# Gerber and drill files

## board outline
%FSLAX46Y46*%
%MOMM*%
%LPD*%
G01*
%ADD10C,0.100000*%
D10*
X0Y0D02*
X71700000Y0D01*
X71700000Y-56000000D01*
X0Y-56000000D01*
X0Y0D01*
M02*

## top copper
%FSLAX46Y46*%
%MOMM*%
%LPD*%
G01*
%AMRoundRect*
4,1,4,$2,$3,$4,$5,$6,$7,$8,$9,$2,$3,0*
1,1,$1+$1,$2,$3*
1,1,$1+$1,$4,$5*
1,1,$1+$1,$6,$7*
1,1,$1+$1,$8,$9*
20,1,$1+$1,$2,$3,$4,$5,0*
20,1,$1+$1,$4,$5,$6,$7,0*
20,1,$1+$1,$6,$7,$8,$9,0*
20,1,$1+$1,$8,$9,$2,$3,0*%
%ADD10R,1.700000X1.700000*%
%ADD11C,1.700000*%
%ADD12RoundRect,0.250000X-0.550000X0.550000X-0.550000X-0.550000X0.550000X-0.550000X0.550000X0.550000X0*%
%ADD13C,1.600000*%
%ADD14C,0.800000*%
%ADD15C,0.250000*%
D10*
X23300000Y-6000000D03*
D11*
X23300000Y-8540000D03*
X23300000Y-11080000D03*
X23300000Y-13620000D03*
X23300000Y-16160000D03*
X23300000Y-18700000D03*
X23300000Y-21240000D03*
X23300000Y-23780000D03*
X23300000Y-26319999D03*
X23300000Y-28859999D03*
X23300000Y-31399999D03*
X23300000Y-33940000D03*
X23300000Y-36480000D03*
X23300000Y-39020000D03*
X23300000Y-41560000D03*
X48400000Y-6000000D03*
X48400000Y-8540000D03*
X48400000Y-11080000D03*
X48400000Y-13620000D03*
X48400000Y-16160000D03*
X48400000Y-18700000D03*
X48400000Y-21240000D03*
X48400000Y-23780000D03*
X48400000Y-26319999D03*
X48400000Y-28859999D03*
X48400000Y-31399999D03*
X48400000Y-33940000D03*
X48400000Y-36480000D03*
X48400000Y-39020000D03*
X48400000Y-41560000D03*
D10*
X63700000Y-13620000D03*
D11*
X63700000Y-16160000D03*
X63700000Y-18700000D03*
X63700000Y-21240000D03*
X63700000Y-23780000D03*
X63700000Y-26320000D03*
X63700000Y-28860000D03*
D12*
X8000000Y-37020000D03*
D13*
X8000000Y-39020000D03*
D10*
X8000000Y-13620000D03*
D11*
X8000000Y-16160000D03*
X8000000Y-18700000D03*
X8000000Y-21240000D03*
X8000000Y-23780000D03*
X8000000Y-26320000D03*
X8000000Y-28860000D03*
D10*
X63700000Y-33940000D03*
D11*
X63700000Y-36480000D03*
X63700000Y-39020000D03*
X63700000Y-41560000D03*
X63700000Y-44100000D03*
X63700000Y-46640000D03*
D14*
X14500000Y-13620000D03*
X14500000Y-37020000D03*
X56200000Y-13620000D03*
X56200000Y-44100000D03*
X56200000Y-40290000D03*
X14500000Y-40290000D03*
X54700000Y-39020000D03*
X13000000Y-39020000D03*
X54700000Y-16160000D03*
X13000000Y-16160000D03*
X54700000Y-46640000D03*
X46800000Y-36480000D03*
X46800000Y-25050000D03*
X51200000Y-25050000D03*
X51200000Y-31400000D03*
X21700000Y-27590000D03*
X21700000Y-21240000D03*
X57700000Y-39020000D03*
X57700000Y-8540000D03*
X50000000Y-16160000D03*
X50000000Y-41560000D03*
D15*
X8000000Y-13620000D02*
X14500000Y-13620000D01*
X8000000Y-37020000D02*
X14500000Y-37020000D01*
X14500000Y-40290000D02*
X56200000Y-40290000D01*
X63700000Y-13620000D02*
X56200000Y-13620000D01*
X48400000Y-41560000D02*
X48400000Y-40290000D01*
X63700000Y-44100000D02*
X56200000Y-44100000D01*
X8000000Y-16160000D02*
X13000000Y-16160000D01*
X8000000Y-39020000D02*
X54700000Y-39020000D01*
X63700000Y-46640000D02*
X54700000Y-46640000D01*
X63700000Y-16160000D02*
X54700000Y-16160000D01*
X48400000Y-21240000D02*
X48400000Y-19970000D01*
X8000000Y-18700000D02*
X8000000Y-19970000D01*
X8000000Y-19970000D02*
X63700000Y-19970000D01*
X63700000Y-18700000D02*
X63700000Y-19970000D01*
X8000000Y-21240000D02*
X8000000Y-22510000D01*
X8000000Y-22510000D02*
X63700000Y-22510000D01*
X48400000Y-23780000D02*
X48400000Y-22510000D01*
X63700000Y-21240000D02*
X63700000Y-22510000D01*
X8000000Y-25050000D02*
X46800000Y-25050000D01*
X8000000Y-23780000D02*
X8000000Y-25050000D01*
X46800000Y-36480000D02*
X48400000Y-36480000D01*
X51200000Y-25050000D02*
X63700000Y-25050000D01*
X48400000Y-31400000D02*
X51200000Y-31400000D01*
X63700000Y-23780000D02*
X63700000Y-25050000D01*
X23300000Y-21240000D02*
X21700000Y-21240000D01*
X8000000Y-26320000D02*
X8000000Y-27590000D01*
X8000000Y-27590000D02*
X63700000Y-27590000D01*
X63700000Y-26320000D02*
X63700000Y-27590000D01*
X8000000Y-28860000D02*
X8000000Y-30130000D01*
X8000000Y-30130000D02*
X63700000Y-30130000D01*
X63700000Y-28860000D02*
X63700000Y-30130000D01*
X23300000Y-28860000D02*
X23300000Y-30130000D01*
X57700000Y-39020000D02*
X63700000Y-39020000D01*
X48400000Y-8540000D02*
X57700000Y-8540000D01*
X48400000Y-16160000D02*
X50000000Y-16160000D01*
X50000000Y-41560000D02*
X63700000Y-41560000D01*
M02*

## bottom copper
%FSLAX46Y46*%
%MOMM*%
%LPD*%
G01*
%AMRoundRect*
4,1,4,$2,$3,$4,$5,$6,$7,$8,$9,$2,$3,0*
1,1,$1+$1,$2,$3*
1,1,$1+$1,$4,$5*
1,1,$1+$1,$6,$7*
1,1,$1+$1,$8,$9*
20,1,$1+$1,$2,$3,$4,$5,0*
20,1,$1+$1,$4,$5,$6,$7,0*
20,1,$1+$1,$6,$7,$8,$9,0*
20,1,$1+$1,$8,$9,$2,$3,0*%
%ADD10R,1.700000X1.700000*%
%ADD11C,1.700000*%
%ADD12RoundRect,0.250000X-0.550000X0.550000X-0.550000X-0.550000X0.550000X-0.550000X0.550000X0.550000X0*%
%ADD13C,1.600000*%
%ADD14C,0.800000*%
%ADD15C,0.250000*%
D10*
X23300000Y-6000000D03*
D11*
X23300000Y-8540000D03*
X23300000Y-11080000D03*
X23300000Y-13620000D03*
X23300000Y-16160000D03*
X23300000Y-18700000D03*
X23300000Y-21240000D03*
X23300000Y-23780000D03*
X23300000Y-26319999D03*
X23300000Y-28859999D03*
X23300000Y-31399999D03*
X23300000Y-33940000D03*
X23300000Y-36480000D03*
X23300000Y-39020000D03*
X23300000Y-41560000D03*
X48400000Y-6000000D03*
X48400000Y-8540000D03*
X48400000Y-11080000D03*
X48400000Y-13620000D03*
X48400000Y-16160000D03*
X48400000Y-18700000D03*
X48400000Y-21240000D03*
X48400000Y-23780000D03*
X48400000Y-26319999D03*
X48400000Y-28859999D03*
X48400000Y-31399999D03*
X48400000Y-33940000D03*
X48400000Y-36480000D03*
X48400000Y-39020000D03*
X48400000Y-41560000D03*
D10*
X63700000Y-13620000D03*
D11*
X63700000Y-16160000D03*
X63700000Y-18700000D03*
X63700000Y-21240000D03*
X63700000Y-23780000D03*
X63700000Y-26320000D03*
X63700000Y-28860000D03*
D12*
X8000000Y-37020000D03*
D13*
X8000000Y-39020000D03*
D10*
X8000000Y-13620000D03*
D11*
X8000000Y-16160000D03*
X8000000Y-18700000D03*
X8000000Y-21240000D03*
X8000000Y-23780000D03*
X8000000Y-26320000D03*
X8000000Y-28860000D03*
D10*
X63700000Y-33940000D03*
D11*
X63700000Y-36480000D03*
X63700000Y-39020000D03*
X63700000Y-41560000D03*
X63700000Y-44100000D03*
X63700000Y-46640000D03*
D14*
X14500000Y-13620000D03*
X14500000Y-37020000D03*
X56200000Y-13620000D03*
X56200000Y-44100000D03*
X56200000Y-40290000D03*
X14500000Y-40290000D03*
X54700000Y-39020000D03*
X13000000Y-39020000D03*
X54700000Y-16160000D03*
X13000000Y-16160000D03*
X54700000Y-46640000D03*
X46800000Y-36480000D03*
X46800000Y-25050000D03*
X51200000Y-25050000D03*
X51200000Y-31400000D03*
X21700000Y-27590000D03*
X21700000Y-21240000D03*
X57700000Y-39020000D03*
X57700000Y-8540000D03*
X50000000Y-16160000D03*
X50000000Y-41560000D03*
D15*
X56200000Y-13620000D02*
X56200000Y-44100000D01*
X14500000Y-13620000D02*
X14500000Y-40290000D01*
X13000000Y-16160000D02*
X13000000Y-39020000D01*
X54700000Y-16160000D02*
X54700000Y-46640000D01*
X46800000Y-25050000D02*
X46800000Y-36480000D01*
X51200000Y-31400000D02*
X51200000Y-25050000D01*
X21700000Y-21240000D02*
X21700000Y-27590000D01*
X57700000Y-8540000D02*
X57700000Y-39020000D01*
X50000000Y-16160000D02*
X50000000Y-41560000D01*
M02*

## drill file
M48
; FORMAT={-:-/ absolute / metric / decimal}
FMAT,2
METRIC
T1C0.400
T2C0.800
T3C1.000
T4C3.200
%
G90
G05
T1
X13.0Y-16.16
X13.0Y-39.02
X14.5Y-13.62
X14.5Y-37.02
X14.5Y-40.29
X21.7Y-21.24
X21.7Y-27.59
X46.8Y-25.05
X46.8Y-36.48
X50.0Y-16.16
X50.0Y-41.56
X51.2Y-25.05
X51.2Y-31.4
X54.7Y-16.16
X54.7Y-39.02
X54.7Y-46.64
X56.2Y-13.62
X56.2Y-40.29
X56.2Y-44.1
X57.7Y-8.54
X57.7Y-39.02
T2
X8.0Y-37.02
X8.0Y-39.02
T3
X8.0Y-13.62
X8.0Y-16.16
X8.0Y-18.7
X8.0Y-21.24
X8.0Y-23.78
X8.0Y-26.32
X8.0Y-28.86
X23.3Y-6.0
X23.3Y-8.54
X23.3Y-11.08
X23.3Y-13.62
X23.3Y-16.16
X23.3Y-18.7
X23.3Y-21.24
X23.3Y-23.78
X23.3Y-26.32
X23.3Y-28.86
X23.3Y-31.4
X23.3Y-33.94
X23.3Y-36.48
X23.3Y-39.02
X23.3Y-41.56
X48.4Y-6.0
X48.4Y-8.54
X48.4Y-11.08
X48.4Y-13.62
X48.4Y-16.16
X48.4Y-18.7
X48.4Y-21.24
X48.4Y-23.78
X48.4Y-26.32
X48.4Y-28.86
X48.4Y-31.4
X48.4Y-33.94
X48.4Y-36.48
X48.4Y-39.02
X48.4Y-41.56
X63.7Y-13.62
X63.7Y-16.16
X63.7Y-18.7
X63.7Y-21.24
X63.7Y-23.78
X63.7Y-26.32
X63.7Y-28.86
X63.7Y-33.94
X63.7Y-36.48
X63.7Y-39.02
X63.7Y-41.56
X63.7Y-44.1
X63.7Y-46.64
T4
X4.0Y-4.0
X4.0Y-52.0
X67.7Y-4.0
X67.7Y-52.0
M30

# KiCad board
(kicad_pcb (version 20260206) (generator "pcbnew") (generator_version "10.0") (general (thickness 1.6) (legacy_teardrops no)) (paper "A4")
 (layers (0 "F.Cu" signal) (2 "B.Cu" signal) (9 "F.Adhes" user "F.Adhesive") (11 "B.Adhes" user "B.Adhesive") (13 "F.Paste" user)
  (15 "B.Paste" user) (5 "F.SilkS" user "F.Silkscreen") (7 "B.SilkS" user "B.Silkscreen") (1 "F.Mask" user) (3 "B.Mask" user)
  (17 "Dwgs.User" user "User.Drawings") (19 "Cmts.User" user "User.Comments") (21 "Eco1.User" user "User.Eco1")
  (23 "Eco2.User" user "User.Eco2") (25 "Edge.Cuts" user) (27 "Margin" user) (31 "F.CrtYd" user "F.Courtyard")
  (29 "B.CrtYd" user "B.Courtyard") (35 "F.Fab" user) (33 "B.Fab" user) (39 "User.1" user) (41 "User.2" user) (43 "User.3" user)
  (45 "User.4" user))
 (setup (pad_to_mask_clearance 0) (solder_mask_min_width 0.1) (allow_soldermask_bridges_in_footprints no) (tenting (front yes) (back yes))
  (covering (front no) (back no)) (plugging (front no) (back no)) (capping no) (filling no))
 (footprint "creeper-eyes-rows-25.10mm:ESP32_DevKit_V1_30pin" (layer "F.Cu") (at 35.85 23.78)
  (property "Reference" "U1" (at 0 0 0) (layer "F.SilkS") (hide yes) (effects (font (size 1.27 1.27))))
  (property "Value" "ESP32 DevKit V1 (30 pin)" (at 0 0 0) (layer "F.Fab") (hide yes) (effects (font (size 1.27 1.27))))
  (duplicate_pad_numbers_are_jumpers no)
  (pad "1" thru_hole rect (at -12.55 -17.78) (size 1.7 1.7) (drill 1) (layers "*.Cu" "*.Mask") (remove_unused_layers no)
   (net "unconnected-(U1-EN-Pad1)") (thermal_bridge_angle 45))
  (pad "2" thru_hole circle (at -12.55 -15.24) (size 1.7 1.7) (drill 1) (layers "*.Cu" "*.Mask") (remove_unused_layers no)
   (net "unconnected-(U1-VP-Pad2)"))
  (pad "3" thru_hole circle (at -12.55 -12.7) (size 1.7 1.7) (drill 1) (layers "*.Cu" "*.Mask") (remove_unused_layers no)
   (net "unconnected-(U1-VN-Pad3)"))
  (pad "4" thru_hole circle (at -12.55 -10.16) (size 1.7 1.7) (drill 1) (layers "*.Cu" "*.Mask") (remove_unused_layers no)
   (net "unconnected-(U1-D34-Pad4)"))
  (pad "5" thru_hole circle (at -12.55 -7.62) (size 1.7 1.7) (drill 1) (layers "*.Cu" "*.Mask") (remove_unused_layers no)
   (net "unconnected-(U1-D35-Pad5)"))
  (pad "6" thru_hole circle (at -12.55 -5.08) (size 1.7 1.7) (drill 1) (layers "*.Cu" "*.Mask") (remove_unused_layers no)
   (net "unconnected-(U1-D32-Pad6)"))
  (pad "7" thru_hole circle (at -12.55 -2.54) (size 1.7 1.7) (drill 1) (layers "*.Cu" "*.Mask") (remove_unused_layers no) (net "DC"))
  (pad "8" thru_hole circle (at -12.55 0) (size 1.7 1.7) (drill 1) (layers "*.Cu" "*.Mask") (remove_unused_layers no)
   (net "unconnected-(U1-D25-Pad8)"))
  (pad "9" thru_hole circle (at -12.55 2.539999) (size 1.7 1.7) (drill 1) (layers "*.Cu" "*.Mask") (remove_unused_layers no)
   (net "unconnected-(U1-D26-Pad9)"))
  (pad "10" thru_hole circle (at -12.55 5.079999) (size 1.7 1.7) (drill 1) (layers "*.Cu" "*.Mask") (remove_unused_layers no) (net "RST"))
  (pad "11" thru_hole circle (at -12.55 7.619999) (size 1.7 1.7) (drill 1) (layers "*.Cu" "*.Mask") (remove_unused_layers no)
   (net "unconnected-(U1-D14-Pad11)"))
  (pad "12" thru_hole circle (at -12.55 10.16) (size 1.7 1.7) (drill 1) (layers "*.Cu" "*.Mask") (remove_unused_layers no)
   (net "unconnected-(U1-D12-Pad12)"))
  (pad "13" thru_hole circle (at -12.55 12.7) (size 1.7 1.7) (drill 1) (layers "*.Cu" "*.Mask") (remove_unused_layers no)
   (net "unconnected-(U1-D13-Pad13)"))
  (pad "14" thru_hole circle (at -12.55 15.24) (size 1.7 1.7) (drill 1) (layers "*.Cu" "*.Mask") (remove_unused_layers no) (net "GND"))
  (pad "15" thru_hole circle (at -12.55 17.78) (size 1.7 1.7) (drill 1) (layers "*.Cu" "*.Mask") (remove_unused_layers no)
   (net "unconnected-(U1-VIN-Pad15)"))
  (pad "16" thru_hole circle (at 12.55 -17.78) (size 1.7 1.7) (drill 1) (layers "*.Cu" "*.Mask") (remove_unused_layers no)
   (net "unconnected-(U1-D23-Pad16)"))
  (pad "17" thru_hole circle (at 12.55 -15.24) (size 1.7 1.7) (drill 1) (layers "*.Cu" "*.Mask") (remove_unused_layers no) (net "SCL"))
  (pad "18" thru_hole circle (at 12.55 -12.7) (size 1.7 1.7) (drill 1) (layers "*.Cu" "*.Mask") (remove_unused_layers no)
   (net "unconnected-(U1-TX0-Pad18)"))
  (pad "19" thru_hole circle (at 12.55 -10.16) (size 1.7 1.7) (drill 1) (layers "*.Cu" "*.Mask") (remove_unused_layers no)
   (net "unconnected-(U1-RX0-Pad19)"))
  (pad "20" thru_hole circle (at 12.55 -7.62) (size 1.7 1.7) (drill 1) (layers "*.Cu" "*.Mask") (remove_unused_layers no) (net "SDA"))
  (pad "21" thru_hole circle (at 12.55 -5.08) (size 1.7 1.7) (drill 1) (layers "*.Cu" "*.Mask") (remove_unused_layers no)
   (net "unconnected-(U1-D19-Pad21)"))
  (pad "22" thru_hole circle (at 12.55 -2.54) (size 1.7 1.7) (drill 1) (layers "*.Cu" "*.Mask") (remove_unused_layers no) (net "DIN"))
  (pad "23" thru_hole circle (at 12.55 0) (size 1.7 1.7) (drill 1) (layers "*.Cu" "*.Mask") (remove_unused_layers no) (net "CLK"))
  (pad "24" thru_hole circle (at 12.55 2.539999) (size 1.7 1.7) (drill 1) (layers "*.Cu" "*.Mask") (remove_unused_layers no)
   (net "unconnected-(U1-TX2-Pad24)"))
  (pad "25" thru_hole circle (at 12.55 5.079999) (size 1.7 1.7) (drill 1) (layers "*.Cu" "*.Mask") (remove_unused_layers no)
   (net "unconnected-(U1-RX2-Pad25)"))
  (pad "26" thru_hole circle (at 12.55 7.619999) (size 1.7 1.7) (drill 1) (layers "*.Cu" "*.Mask") (remove_unused_layers no) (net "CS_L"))
  (pad "27" thru_hole circle (at 12.55 10.16) (size 1.7 1.7) (drill 1) (layers "*.Cu" "*.Mask") (remove_unused_layers no)
   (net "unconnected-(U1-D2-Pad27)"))
  (pad "28" thru_hole circle (at 12.55 12.7) (size 1.7 1.7) (drill 1) (layers "*.Cu" "*.Mask") (remove_unused_layers no) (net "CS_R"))
  (pad "29" thru_hole circle (at 12.55 15.24) (size 1.7 1.7) (drill 1) (layers "*.Cu" "*.Mask") (remove_unused_layers no) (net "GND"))
  (pad "30" thru_hole circle (at 12.55 17.78) (size 1.7 1.7) (drill 1) (layers "*.Cu" "*.Mask") (remove_unused_layers no) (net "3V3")))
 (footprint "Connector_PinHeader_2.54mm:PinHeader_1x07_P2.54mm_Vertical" (layer "F.Cu") (at 63.7 13.62)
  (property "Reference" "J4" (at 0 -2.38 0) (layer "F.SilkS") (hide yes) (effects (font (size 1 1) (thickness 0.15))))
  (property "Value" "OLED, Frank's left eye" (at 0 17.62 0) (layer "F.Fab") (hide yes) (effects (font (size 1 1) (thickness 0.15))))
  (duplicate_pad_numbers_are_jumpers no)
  (pad "1" thru_hole rect (at 0 0) (size 1.7 1.7) (drill 1) (layers "*.Cu" "*.Mask") (remove_unused_layers no) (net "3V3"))
  (pad "2" thru_hole circle (at 0 2.54) (size 1.7 1.7) (drill 1) (layers "*.Cu" "*.Mask") (remove_unused_layers no) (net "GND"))
  (pad "3" thru_hole circle (at 0 5.08) (size 1.7 1.7) (drill 1) (layers "*.Cu" "*.Mask") (remove_unused_layers no) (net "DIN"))
  (pad "4" thru_hole circle (at 0 7.62) (size 1.7 1.7) (drill 1) (layers "*.Cu" "*.Mask") (remove_unused_layers no) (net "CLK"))
  (pad "5" thru_hole circle (at 0 10.16) (size 1.7 1.7) (drill 1) (layers "*.Cu" "*.Mask") (remove_unused_layers no) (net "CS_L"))
  (pad "6" thru_hole circle (at 0 12.7) (size 1.7 1.7) (drill 1) (layers "*.Cu" "*.Mask") (remove_unused_layers no) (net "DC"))
  (pad "7" thru_hole circle (at 0 15.24) (size 1.7 1.7) (drill 1) (layers "*.Cu" "*.Mask") (remove_unused_layers no) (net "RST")))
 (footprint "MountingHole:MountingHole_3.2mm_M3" (layer "F.Cu") (at 67.7 4)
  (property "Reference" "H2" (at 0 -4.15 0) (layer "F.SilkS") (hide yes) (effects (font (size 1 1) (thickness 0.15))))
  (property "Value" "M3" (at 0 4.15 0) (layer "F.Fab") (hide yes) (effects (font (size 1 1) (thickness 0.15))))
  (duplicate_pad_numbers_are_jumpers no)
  (pad "" np_thru_hole circle (at 0 0) (size 3.2 3.2) (drill 3.2) (layers "*.Cu" "*.Mask")))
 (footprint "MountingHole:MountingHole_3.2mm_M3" (layer "F.Cu") (at 4 52)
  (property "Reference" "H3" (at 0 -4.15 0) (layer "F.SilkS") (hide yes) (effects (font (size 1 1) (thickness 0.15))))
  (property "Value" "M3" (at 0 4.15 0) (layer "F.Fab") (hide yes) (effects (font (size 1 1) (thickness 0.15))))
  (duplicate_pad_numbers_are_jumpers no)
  (pad "" np_thru_hole circle (at 0 0) (size 3.2 3.2) (drill 3.2) (layers "*.Cu" "*.Mask")))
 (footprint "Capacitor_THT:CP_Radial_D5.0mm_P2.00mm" (layer "F.Cu") (at 8 37.02 -90)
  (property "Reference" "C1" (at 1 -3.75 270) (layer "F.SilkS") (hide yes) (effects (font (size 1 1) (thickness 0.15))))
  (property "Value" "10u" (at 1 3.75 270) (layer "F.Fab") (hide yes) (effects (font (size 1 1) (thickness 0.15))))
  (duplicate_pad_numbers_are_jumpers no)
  (pad "1" thru_hole roundrect (at 0 0 270) (size 1.6 1.6) (drill 0.8) (layers "*.Cu" "*.Mask") (remove_unused_layers no)
   (roundrect_rratio 0.15625) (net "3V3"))
  (pad "2" thru_hole circle (at 2 0 270) (size 1.6 1.6) (drill 0.8) (layers "*.Cu" "*.Mask") (remove_unused_layers no) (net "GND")))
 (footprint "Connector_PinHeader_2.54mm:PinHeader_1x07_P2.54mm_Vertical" (layer "F.Cu") (at 8 13.62)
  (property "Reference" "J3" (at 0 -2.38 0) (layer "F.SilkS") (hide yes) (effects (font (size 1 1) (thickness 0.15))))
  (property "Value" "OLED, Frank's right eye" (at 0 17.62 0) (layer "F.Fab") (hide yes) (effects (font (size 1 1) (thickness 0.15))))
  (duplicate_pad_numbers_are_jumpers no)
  (pad "1" thru_hole rect (at 0 0) (size 1.7 1.7) (drill 1) (layers "*.Cu" "*.Mask") (remove_unused_layers no) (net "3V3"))
  (pad "2" thru_hole circle (at 0 2.54) (size 1.7 1.7) (drill 1) (layers "*.Cu" "*.Mask") (remove_unused_layers no) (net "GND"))
  (pad "3" thru_hole circle (at 0 5.08) (size 1.7 1.7) (drill 1) (layers "*.Cu" "*.Mask") (remove_unused_layers no) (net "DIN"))
  (pad "4" thru_hole circle (at 0 7.62) (size 1.7 1.7) (drill 1) (layers "*.Cu" "*.Mask") (remove_unused_layers no) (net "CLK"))
  (pad "5" thru_hole circle (at 0 10.16) (size 1.7 1.7) (drill 1) (layers "*.Cu" "*.Mask") (remove_unused_layers no) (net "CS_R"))
  (pad "6" thru_hole circle (at 0 12.7) (size 1.7 1.7) (drill 1) (layers "*.Cu" "*.Mask") (remove_unused_layers no) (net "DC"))
  (pad "7" thru_hole circle (at 0 15.24) (size 1.7 1.7) (drill 1) (layers "*.Cu" "*.Mask") (remove_unused_layers no) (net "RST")))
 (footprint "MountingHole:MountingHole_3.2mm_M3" (layer "F.Cu") (at 67.7 52)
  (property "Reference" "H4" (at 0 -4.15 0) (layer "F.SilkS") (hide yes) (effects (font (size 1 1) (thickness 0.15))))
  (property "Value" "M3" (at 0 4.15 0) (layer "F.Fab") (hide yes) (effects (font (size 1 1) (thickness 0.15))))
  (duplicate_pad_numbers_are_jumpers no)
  (pad "" np_thru_hole circle (at 0 0) (size 3.2 3.2) (drill 3.2) (layers "*.Cu" "*.Mask")))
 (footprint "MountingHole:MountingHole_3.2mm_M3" (layer "F.Cu") (at 4 4)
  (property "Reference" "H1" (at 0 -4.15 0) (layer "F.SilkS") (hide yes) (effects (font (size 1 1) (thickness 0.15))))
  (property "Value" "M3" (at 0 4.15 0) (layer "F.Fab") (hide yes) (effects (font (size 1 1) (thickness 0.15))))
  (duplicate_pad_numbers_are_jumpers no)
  (pad "" np_thru_hole circle (at 0 0) (size 3.2 3.2) (drill 3.2) (layers "*.Cu" "*.Mask")))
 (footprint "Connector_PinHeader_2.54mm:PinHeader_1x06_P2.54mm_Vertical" (layer "F.Cu") (at 63.7 33.94)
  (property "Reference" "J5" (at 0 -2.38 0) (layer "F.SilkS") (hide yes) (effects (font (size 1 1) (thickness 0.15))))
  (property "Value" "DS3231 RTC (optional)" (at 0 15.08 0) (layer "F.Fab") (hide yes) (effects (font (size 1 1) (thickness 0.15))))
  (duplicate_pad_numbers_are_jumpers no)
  (pad "1" thru_hole rect (at 0 0) (size 1.7 1.7) (drill 1) (layers "*.Cu" "*.Mask") (remove_unused_layers no)
   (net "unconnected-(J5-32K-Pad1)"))
  (pad "2" thru_hole circle (at 0 2.54) (size 1.7 1.7) (drill 1) (layers "*.Cu" "*.Mask") (remove_unused_layers no)
   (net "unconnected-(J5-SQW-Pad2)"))
  (pad "3" thru_hole circle (at 0 5.08) (size 1.7 1.7) (drill 1) (layers "*.Cu" "*.Mask") (remove_unused_layers no) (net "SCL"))
  (pad "4" thru_hole circle (at 0 7.62) (size 1.7 1.7) (drill 1) (layers "*.Cu" "*.Mask") (remove_unused_layers no) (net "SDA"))
  (pad "5" thru_hole circle (at 0 10.16) (size 1.7 1.7) (drill 1) (layers "*.Cu" "*.Mask") (remove_unused_layers no) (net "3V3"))
  (pad "6" thru_hole circle (at 0 12.7) (size 1.7 1.7) (drill 1) (layers "*.Cu" "*.Mask") (remove_unused_layers no) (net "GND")))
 (gr_rect (start 0 0) (end 71.7 56) (stroke (width 0.1) (type default)) (fill no) (layer "Edge.Cuts"))
 (segment (start 8 13.62) (end 14.5 13.62) (width 0.25) (layer "F.Cu") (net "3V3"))
 (segment (start 8 37.02) (end 14.5 37.02) (width 0.25) (layer "F.Cu") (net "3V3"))
 (segment (start 14.5 40.29) (end 56.2 40.29) (width 0.25) (layer "F.Cu") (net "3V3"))
 (segment (start 63.7 13.62) (end 56.2 13.62) (width 0.25) (layer "F.Cu") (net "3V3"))
 (segment (start 48.4 41.56) (end 48.4 40.29) (width 0.25) (layer "F.Cu") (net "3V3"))
 (segment (start 63.7 44.1) (end 56.2 44.1) (width 0.25) (layer "F.Cu") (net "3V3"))
 (via (at 14.5 13.62) (size 0.8) (drill 0.4) (layers "F.Cu" "B.Cu") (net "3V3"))
 (via (at 14.5 37.02) (size 0.8) (drill 0.4) (layers "F.Cu" "B.Cu") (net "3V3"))
 (via (at 56.2 13.62) (size 0.8) (drill 0.4) (layers "F.Cu" "B.Cu") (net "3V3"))
 (via (at 56.2 44.1) (size 0.8) (drill 0.4) (layers "F.Cu" "B.Cu") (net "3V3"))
 (via (at 56.2 40.29) (size 0.8) (drill 0.4) (layers "F.Cu" "B.Cu") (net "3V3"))
 (via (at 14.5 40.29) (size 0.8) (drill 0.4) (layers "F.Cu" "B.Cu") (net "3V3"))
 (segment (start 56.2 13.62) (end 56.2 44.1) (width 0.25) (layer "B.Cu") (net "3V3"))
 (segment (start 14.5 13.62) (end 14.5 40.29) (width 0.25) (layer "B.Cu") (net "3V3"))
 (segment (start 8 16.16) (end 13 16.16) (width 0.25) (layer "F.Cu") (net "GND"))
 (segment (start 8 39.02) (end 54.7 39.02) (width 0.25) (layer "F.Cu") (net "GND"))
 (segment (start 63.7 46.64) (end 54.7 46.64) (width 0.25) (layer "F.Cu") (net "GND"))
 (segment (start 63.7 16.16) (end 54.7 16.16) (width 0.25) (layer "F.Cu") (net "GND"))
 (via (at 54.7 39.02) (size 0.8) (drill 0.4) (layers "F.Cu" "B.Cu") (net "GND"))
 (via (at 13 39.02) (size 0.8) (drill 0.4) (layers "F.Cu" "B.Cu") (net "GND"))
 (via (at 54.7 16.16) (size 0.8) (drill 0.4) (layers "F.Cu" "B.Cu") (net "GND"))
 (via (at 13 16.16) (size 0.8) (drill 0.4) (layers "F.Cu" "B.Cu") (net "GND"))
 (via (at 54.7 46.64) (size 0.8) (drill 0.4) (layers "F.Cu" "B.Cu") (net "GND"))
 (segment (start 13 16.16) (end 13 39.02) (width 0.25) (layer "B.Cu") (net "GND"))
 (segment (start 54.7 16.16) (end 54.7 46.64) (width 0.25) (layer "B.Cu") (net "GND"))
 (segment (start 48.4 21.24) (end 48.4 19.97) (width 0.25) (layer "F.Cu") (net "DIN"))
 (segment (start 8 18.7) (end 8 19.97) (width 0.25) (layer "F.Cu") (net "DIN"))
 (segment (start 8 19.97) (end 63.7 19.97) (width 0.25) (layer "F.Cu") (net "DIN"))
 (segment (start 63.7 18.7) (end 63.7 19.97) (width 0.25) (layer "F.Cu") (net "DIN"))
 (segment (start 8 21.24) (end 8 22.51) (width 0.25) (layer "F.Cu") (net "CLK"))
 (segment (start 8 22.51) (end 63.7 22.51) (width 0.25) (layer "F.Cu") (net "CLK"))
 (segment (start 48.4 23.78) (end 48.4 22.51) (width 0.25) (layer "F.Cu") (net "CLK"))
 (segment (start 63.7 21.24) (end 63.7 22.51) (width 0.25) (layer "F.Cu") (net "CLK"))
 (segment (start 8 25.05) (end 46.8 25.05) (width 0.25) (layer "F.Cu") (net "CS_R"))
 (segment (start 8 23.78) (end 8 25.05) (width 0.25) (layer "F.Cu") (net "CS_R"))
 (segment (start 46.8 36.48) (end 48.4 36.48) (width 0.25) (layer "F.Cu") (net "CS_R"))
 (via (at 46.8 36.48) (size 0.8) (drill 0.4) (layers "F.Cu" "B.Cu") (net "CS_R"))
 (via (at 46.8 25.05) (size 0.8) (drill 0.4) (layers "F.Cu" "B.Cu") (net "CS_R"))
 (segment (start 46.8 25.05) (end 46.8 36.48) (width 0.25) (layer "B.Cu") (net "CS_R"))
 (segment (start 51.2 25.05) (end 63.7 25.05) (width 0.25) (layer "F.Cu") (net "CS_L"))
 (segment (start 48.4 31.4) (end 51.2 31.4) (width 0.25) (layer "F.Cu") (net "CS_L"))
 (segment (start 63.7 23.78) (end 63.7 25.05) (width 0.25) (layer "F.Cu") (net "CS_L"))
 (via (at 51.2 25.05) (size 0.8) (drill 0.4) (layers "F.Cu" "B.Cu") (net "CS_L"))
 (via (at 51.2 31.4) (size 0.8) (drill 0.4) (layers "F.Cu" "B.Cu") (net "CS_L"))
 (segment (start 51.2 31.4) (end 51.2 25.05) (width 0.25) (layer "B.Cu") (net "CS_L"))
 (segment (start 23.3 21.24) (end 21.7 21.24) (width 0.25) (layer "F.Cu") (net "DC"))
 (segment (start 8 26.32) (end 8 27.59) (width 0.25) (layer "F.Cu") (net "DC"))
 (segment (start 8 27.59) (end 63.7 27.59) (width 0.25) (layer "F.Cu") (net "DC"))
 (segment (start 63.7 26.32) (end 63.7 27.59) (width 0.25) (layer "F.Cu") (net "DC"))
 (via (at 21.7 27.59) (size 0.8) (drill 0.4) (layers "F.Cu" "B.Cu") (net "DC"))
 (via (at 21.7 21.24) (size 0.8) (drill 0.4) (layers "F.Cu" "B.Cu") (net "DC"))
 (segment (start 21.7 21.24) (end 21.7 27.59) (width 0.25) (layer "B.Cu") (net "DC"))
 (segment (start 8 28.86) (end 8 30.13) (width 0.25) (layer "F.Cu") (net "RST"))
 (segment (start 8 30.13) (end 63.7 30.13) (width 0.25) (layer "F.Cu") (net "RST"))
 (segment (start 63.7 28.86) (end 63.7 30.13) (width 0.25) (layer "F.Cu") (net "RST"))
 (segment (start 23.3 28.86) (end 23.3 30.13) (width 0.25) (layer "F.Cu") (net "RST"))
 (segment (start 57.7 39.02) (end 63.7 39.02) (width 0.25) (layer "F.Cu") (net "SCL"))
 (segment (start 48.4 8.54) (end 57.7 8.54) (width 0.25) (layer "F.Cu") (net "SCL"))
 (via (at 57.7 39.02) (size 0.8) (drill 0.4) (layers "F.Cu" "B.Cu") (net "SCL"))
 (via (at 57.7 8.54) (size 0.8) (drill 0.4) (layers "F.Cu" "B.Cu") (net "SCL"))
 (segment (start 57.7 8.54) (end 57.7 39.02) (width 0.25) (layer "B.Cu") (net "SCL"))
 (segment (start 48.4 16.16) (end 50 16.16) (width 0.25) (layer "F.Cu") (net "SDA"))
 (segment (start 50 41.56) (end 63.7 41.56) (width 0.25) (layer "F.Cu") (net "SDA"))
 (via (at 50 16.16) (size 0.8) (drill 0.4) (layers "F.Cu" "B.Cu") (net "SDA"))
 (via (at 50 41.56) (size 0.8) (drill 0.4) (layers "F.Cu" "B.Cu") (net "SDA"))
 (segment (start 50 16.16) (end 50 41.56) (width 0.25) (layer "B.Cu") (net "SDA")))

